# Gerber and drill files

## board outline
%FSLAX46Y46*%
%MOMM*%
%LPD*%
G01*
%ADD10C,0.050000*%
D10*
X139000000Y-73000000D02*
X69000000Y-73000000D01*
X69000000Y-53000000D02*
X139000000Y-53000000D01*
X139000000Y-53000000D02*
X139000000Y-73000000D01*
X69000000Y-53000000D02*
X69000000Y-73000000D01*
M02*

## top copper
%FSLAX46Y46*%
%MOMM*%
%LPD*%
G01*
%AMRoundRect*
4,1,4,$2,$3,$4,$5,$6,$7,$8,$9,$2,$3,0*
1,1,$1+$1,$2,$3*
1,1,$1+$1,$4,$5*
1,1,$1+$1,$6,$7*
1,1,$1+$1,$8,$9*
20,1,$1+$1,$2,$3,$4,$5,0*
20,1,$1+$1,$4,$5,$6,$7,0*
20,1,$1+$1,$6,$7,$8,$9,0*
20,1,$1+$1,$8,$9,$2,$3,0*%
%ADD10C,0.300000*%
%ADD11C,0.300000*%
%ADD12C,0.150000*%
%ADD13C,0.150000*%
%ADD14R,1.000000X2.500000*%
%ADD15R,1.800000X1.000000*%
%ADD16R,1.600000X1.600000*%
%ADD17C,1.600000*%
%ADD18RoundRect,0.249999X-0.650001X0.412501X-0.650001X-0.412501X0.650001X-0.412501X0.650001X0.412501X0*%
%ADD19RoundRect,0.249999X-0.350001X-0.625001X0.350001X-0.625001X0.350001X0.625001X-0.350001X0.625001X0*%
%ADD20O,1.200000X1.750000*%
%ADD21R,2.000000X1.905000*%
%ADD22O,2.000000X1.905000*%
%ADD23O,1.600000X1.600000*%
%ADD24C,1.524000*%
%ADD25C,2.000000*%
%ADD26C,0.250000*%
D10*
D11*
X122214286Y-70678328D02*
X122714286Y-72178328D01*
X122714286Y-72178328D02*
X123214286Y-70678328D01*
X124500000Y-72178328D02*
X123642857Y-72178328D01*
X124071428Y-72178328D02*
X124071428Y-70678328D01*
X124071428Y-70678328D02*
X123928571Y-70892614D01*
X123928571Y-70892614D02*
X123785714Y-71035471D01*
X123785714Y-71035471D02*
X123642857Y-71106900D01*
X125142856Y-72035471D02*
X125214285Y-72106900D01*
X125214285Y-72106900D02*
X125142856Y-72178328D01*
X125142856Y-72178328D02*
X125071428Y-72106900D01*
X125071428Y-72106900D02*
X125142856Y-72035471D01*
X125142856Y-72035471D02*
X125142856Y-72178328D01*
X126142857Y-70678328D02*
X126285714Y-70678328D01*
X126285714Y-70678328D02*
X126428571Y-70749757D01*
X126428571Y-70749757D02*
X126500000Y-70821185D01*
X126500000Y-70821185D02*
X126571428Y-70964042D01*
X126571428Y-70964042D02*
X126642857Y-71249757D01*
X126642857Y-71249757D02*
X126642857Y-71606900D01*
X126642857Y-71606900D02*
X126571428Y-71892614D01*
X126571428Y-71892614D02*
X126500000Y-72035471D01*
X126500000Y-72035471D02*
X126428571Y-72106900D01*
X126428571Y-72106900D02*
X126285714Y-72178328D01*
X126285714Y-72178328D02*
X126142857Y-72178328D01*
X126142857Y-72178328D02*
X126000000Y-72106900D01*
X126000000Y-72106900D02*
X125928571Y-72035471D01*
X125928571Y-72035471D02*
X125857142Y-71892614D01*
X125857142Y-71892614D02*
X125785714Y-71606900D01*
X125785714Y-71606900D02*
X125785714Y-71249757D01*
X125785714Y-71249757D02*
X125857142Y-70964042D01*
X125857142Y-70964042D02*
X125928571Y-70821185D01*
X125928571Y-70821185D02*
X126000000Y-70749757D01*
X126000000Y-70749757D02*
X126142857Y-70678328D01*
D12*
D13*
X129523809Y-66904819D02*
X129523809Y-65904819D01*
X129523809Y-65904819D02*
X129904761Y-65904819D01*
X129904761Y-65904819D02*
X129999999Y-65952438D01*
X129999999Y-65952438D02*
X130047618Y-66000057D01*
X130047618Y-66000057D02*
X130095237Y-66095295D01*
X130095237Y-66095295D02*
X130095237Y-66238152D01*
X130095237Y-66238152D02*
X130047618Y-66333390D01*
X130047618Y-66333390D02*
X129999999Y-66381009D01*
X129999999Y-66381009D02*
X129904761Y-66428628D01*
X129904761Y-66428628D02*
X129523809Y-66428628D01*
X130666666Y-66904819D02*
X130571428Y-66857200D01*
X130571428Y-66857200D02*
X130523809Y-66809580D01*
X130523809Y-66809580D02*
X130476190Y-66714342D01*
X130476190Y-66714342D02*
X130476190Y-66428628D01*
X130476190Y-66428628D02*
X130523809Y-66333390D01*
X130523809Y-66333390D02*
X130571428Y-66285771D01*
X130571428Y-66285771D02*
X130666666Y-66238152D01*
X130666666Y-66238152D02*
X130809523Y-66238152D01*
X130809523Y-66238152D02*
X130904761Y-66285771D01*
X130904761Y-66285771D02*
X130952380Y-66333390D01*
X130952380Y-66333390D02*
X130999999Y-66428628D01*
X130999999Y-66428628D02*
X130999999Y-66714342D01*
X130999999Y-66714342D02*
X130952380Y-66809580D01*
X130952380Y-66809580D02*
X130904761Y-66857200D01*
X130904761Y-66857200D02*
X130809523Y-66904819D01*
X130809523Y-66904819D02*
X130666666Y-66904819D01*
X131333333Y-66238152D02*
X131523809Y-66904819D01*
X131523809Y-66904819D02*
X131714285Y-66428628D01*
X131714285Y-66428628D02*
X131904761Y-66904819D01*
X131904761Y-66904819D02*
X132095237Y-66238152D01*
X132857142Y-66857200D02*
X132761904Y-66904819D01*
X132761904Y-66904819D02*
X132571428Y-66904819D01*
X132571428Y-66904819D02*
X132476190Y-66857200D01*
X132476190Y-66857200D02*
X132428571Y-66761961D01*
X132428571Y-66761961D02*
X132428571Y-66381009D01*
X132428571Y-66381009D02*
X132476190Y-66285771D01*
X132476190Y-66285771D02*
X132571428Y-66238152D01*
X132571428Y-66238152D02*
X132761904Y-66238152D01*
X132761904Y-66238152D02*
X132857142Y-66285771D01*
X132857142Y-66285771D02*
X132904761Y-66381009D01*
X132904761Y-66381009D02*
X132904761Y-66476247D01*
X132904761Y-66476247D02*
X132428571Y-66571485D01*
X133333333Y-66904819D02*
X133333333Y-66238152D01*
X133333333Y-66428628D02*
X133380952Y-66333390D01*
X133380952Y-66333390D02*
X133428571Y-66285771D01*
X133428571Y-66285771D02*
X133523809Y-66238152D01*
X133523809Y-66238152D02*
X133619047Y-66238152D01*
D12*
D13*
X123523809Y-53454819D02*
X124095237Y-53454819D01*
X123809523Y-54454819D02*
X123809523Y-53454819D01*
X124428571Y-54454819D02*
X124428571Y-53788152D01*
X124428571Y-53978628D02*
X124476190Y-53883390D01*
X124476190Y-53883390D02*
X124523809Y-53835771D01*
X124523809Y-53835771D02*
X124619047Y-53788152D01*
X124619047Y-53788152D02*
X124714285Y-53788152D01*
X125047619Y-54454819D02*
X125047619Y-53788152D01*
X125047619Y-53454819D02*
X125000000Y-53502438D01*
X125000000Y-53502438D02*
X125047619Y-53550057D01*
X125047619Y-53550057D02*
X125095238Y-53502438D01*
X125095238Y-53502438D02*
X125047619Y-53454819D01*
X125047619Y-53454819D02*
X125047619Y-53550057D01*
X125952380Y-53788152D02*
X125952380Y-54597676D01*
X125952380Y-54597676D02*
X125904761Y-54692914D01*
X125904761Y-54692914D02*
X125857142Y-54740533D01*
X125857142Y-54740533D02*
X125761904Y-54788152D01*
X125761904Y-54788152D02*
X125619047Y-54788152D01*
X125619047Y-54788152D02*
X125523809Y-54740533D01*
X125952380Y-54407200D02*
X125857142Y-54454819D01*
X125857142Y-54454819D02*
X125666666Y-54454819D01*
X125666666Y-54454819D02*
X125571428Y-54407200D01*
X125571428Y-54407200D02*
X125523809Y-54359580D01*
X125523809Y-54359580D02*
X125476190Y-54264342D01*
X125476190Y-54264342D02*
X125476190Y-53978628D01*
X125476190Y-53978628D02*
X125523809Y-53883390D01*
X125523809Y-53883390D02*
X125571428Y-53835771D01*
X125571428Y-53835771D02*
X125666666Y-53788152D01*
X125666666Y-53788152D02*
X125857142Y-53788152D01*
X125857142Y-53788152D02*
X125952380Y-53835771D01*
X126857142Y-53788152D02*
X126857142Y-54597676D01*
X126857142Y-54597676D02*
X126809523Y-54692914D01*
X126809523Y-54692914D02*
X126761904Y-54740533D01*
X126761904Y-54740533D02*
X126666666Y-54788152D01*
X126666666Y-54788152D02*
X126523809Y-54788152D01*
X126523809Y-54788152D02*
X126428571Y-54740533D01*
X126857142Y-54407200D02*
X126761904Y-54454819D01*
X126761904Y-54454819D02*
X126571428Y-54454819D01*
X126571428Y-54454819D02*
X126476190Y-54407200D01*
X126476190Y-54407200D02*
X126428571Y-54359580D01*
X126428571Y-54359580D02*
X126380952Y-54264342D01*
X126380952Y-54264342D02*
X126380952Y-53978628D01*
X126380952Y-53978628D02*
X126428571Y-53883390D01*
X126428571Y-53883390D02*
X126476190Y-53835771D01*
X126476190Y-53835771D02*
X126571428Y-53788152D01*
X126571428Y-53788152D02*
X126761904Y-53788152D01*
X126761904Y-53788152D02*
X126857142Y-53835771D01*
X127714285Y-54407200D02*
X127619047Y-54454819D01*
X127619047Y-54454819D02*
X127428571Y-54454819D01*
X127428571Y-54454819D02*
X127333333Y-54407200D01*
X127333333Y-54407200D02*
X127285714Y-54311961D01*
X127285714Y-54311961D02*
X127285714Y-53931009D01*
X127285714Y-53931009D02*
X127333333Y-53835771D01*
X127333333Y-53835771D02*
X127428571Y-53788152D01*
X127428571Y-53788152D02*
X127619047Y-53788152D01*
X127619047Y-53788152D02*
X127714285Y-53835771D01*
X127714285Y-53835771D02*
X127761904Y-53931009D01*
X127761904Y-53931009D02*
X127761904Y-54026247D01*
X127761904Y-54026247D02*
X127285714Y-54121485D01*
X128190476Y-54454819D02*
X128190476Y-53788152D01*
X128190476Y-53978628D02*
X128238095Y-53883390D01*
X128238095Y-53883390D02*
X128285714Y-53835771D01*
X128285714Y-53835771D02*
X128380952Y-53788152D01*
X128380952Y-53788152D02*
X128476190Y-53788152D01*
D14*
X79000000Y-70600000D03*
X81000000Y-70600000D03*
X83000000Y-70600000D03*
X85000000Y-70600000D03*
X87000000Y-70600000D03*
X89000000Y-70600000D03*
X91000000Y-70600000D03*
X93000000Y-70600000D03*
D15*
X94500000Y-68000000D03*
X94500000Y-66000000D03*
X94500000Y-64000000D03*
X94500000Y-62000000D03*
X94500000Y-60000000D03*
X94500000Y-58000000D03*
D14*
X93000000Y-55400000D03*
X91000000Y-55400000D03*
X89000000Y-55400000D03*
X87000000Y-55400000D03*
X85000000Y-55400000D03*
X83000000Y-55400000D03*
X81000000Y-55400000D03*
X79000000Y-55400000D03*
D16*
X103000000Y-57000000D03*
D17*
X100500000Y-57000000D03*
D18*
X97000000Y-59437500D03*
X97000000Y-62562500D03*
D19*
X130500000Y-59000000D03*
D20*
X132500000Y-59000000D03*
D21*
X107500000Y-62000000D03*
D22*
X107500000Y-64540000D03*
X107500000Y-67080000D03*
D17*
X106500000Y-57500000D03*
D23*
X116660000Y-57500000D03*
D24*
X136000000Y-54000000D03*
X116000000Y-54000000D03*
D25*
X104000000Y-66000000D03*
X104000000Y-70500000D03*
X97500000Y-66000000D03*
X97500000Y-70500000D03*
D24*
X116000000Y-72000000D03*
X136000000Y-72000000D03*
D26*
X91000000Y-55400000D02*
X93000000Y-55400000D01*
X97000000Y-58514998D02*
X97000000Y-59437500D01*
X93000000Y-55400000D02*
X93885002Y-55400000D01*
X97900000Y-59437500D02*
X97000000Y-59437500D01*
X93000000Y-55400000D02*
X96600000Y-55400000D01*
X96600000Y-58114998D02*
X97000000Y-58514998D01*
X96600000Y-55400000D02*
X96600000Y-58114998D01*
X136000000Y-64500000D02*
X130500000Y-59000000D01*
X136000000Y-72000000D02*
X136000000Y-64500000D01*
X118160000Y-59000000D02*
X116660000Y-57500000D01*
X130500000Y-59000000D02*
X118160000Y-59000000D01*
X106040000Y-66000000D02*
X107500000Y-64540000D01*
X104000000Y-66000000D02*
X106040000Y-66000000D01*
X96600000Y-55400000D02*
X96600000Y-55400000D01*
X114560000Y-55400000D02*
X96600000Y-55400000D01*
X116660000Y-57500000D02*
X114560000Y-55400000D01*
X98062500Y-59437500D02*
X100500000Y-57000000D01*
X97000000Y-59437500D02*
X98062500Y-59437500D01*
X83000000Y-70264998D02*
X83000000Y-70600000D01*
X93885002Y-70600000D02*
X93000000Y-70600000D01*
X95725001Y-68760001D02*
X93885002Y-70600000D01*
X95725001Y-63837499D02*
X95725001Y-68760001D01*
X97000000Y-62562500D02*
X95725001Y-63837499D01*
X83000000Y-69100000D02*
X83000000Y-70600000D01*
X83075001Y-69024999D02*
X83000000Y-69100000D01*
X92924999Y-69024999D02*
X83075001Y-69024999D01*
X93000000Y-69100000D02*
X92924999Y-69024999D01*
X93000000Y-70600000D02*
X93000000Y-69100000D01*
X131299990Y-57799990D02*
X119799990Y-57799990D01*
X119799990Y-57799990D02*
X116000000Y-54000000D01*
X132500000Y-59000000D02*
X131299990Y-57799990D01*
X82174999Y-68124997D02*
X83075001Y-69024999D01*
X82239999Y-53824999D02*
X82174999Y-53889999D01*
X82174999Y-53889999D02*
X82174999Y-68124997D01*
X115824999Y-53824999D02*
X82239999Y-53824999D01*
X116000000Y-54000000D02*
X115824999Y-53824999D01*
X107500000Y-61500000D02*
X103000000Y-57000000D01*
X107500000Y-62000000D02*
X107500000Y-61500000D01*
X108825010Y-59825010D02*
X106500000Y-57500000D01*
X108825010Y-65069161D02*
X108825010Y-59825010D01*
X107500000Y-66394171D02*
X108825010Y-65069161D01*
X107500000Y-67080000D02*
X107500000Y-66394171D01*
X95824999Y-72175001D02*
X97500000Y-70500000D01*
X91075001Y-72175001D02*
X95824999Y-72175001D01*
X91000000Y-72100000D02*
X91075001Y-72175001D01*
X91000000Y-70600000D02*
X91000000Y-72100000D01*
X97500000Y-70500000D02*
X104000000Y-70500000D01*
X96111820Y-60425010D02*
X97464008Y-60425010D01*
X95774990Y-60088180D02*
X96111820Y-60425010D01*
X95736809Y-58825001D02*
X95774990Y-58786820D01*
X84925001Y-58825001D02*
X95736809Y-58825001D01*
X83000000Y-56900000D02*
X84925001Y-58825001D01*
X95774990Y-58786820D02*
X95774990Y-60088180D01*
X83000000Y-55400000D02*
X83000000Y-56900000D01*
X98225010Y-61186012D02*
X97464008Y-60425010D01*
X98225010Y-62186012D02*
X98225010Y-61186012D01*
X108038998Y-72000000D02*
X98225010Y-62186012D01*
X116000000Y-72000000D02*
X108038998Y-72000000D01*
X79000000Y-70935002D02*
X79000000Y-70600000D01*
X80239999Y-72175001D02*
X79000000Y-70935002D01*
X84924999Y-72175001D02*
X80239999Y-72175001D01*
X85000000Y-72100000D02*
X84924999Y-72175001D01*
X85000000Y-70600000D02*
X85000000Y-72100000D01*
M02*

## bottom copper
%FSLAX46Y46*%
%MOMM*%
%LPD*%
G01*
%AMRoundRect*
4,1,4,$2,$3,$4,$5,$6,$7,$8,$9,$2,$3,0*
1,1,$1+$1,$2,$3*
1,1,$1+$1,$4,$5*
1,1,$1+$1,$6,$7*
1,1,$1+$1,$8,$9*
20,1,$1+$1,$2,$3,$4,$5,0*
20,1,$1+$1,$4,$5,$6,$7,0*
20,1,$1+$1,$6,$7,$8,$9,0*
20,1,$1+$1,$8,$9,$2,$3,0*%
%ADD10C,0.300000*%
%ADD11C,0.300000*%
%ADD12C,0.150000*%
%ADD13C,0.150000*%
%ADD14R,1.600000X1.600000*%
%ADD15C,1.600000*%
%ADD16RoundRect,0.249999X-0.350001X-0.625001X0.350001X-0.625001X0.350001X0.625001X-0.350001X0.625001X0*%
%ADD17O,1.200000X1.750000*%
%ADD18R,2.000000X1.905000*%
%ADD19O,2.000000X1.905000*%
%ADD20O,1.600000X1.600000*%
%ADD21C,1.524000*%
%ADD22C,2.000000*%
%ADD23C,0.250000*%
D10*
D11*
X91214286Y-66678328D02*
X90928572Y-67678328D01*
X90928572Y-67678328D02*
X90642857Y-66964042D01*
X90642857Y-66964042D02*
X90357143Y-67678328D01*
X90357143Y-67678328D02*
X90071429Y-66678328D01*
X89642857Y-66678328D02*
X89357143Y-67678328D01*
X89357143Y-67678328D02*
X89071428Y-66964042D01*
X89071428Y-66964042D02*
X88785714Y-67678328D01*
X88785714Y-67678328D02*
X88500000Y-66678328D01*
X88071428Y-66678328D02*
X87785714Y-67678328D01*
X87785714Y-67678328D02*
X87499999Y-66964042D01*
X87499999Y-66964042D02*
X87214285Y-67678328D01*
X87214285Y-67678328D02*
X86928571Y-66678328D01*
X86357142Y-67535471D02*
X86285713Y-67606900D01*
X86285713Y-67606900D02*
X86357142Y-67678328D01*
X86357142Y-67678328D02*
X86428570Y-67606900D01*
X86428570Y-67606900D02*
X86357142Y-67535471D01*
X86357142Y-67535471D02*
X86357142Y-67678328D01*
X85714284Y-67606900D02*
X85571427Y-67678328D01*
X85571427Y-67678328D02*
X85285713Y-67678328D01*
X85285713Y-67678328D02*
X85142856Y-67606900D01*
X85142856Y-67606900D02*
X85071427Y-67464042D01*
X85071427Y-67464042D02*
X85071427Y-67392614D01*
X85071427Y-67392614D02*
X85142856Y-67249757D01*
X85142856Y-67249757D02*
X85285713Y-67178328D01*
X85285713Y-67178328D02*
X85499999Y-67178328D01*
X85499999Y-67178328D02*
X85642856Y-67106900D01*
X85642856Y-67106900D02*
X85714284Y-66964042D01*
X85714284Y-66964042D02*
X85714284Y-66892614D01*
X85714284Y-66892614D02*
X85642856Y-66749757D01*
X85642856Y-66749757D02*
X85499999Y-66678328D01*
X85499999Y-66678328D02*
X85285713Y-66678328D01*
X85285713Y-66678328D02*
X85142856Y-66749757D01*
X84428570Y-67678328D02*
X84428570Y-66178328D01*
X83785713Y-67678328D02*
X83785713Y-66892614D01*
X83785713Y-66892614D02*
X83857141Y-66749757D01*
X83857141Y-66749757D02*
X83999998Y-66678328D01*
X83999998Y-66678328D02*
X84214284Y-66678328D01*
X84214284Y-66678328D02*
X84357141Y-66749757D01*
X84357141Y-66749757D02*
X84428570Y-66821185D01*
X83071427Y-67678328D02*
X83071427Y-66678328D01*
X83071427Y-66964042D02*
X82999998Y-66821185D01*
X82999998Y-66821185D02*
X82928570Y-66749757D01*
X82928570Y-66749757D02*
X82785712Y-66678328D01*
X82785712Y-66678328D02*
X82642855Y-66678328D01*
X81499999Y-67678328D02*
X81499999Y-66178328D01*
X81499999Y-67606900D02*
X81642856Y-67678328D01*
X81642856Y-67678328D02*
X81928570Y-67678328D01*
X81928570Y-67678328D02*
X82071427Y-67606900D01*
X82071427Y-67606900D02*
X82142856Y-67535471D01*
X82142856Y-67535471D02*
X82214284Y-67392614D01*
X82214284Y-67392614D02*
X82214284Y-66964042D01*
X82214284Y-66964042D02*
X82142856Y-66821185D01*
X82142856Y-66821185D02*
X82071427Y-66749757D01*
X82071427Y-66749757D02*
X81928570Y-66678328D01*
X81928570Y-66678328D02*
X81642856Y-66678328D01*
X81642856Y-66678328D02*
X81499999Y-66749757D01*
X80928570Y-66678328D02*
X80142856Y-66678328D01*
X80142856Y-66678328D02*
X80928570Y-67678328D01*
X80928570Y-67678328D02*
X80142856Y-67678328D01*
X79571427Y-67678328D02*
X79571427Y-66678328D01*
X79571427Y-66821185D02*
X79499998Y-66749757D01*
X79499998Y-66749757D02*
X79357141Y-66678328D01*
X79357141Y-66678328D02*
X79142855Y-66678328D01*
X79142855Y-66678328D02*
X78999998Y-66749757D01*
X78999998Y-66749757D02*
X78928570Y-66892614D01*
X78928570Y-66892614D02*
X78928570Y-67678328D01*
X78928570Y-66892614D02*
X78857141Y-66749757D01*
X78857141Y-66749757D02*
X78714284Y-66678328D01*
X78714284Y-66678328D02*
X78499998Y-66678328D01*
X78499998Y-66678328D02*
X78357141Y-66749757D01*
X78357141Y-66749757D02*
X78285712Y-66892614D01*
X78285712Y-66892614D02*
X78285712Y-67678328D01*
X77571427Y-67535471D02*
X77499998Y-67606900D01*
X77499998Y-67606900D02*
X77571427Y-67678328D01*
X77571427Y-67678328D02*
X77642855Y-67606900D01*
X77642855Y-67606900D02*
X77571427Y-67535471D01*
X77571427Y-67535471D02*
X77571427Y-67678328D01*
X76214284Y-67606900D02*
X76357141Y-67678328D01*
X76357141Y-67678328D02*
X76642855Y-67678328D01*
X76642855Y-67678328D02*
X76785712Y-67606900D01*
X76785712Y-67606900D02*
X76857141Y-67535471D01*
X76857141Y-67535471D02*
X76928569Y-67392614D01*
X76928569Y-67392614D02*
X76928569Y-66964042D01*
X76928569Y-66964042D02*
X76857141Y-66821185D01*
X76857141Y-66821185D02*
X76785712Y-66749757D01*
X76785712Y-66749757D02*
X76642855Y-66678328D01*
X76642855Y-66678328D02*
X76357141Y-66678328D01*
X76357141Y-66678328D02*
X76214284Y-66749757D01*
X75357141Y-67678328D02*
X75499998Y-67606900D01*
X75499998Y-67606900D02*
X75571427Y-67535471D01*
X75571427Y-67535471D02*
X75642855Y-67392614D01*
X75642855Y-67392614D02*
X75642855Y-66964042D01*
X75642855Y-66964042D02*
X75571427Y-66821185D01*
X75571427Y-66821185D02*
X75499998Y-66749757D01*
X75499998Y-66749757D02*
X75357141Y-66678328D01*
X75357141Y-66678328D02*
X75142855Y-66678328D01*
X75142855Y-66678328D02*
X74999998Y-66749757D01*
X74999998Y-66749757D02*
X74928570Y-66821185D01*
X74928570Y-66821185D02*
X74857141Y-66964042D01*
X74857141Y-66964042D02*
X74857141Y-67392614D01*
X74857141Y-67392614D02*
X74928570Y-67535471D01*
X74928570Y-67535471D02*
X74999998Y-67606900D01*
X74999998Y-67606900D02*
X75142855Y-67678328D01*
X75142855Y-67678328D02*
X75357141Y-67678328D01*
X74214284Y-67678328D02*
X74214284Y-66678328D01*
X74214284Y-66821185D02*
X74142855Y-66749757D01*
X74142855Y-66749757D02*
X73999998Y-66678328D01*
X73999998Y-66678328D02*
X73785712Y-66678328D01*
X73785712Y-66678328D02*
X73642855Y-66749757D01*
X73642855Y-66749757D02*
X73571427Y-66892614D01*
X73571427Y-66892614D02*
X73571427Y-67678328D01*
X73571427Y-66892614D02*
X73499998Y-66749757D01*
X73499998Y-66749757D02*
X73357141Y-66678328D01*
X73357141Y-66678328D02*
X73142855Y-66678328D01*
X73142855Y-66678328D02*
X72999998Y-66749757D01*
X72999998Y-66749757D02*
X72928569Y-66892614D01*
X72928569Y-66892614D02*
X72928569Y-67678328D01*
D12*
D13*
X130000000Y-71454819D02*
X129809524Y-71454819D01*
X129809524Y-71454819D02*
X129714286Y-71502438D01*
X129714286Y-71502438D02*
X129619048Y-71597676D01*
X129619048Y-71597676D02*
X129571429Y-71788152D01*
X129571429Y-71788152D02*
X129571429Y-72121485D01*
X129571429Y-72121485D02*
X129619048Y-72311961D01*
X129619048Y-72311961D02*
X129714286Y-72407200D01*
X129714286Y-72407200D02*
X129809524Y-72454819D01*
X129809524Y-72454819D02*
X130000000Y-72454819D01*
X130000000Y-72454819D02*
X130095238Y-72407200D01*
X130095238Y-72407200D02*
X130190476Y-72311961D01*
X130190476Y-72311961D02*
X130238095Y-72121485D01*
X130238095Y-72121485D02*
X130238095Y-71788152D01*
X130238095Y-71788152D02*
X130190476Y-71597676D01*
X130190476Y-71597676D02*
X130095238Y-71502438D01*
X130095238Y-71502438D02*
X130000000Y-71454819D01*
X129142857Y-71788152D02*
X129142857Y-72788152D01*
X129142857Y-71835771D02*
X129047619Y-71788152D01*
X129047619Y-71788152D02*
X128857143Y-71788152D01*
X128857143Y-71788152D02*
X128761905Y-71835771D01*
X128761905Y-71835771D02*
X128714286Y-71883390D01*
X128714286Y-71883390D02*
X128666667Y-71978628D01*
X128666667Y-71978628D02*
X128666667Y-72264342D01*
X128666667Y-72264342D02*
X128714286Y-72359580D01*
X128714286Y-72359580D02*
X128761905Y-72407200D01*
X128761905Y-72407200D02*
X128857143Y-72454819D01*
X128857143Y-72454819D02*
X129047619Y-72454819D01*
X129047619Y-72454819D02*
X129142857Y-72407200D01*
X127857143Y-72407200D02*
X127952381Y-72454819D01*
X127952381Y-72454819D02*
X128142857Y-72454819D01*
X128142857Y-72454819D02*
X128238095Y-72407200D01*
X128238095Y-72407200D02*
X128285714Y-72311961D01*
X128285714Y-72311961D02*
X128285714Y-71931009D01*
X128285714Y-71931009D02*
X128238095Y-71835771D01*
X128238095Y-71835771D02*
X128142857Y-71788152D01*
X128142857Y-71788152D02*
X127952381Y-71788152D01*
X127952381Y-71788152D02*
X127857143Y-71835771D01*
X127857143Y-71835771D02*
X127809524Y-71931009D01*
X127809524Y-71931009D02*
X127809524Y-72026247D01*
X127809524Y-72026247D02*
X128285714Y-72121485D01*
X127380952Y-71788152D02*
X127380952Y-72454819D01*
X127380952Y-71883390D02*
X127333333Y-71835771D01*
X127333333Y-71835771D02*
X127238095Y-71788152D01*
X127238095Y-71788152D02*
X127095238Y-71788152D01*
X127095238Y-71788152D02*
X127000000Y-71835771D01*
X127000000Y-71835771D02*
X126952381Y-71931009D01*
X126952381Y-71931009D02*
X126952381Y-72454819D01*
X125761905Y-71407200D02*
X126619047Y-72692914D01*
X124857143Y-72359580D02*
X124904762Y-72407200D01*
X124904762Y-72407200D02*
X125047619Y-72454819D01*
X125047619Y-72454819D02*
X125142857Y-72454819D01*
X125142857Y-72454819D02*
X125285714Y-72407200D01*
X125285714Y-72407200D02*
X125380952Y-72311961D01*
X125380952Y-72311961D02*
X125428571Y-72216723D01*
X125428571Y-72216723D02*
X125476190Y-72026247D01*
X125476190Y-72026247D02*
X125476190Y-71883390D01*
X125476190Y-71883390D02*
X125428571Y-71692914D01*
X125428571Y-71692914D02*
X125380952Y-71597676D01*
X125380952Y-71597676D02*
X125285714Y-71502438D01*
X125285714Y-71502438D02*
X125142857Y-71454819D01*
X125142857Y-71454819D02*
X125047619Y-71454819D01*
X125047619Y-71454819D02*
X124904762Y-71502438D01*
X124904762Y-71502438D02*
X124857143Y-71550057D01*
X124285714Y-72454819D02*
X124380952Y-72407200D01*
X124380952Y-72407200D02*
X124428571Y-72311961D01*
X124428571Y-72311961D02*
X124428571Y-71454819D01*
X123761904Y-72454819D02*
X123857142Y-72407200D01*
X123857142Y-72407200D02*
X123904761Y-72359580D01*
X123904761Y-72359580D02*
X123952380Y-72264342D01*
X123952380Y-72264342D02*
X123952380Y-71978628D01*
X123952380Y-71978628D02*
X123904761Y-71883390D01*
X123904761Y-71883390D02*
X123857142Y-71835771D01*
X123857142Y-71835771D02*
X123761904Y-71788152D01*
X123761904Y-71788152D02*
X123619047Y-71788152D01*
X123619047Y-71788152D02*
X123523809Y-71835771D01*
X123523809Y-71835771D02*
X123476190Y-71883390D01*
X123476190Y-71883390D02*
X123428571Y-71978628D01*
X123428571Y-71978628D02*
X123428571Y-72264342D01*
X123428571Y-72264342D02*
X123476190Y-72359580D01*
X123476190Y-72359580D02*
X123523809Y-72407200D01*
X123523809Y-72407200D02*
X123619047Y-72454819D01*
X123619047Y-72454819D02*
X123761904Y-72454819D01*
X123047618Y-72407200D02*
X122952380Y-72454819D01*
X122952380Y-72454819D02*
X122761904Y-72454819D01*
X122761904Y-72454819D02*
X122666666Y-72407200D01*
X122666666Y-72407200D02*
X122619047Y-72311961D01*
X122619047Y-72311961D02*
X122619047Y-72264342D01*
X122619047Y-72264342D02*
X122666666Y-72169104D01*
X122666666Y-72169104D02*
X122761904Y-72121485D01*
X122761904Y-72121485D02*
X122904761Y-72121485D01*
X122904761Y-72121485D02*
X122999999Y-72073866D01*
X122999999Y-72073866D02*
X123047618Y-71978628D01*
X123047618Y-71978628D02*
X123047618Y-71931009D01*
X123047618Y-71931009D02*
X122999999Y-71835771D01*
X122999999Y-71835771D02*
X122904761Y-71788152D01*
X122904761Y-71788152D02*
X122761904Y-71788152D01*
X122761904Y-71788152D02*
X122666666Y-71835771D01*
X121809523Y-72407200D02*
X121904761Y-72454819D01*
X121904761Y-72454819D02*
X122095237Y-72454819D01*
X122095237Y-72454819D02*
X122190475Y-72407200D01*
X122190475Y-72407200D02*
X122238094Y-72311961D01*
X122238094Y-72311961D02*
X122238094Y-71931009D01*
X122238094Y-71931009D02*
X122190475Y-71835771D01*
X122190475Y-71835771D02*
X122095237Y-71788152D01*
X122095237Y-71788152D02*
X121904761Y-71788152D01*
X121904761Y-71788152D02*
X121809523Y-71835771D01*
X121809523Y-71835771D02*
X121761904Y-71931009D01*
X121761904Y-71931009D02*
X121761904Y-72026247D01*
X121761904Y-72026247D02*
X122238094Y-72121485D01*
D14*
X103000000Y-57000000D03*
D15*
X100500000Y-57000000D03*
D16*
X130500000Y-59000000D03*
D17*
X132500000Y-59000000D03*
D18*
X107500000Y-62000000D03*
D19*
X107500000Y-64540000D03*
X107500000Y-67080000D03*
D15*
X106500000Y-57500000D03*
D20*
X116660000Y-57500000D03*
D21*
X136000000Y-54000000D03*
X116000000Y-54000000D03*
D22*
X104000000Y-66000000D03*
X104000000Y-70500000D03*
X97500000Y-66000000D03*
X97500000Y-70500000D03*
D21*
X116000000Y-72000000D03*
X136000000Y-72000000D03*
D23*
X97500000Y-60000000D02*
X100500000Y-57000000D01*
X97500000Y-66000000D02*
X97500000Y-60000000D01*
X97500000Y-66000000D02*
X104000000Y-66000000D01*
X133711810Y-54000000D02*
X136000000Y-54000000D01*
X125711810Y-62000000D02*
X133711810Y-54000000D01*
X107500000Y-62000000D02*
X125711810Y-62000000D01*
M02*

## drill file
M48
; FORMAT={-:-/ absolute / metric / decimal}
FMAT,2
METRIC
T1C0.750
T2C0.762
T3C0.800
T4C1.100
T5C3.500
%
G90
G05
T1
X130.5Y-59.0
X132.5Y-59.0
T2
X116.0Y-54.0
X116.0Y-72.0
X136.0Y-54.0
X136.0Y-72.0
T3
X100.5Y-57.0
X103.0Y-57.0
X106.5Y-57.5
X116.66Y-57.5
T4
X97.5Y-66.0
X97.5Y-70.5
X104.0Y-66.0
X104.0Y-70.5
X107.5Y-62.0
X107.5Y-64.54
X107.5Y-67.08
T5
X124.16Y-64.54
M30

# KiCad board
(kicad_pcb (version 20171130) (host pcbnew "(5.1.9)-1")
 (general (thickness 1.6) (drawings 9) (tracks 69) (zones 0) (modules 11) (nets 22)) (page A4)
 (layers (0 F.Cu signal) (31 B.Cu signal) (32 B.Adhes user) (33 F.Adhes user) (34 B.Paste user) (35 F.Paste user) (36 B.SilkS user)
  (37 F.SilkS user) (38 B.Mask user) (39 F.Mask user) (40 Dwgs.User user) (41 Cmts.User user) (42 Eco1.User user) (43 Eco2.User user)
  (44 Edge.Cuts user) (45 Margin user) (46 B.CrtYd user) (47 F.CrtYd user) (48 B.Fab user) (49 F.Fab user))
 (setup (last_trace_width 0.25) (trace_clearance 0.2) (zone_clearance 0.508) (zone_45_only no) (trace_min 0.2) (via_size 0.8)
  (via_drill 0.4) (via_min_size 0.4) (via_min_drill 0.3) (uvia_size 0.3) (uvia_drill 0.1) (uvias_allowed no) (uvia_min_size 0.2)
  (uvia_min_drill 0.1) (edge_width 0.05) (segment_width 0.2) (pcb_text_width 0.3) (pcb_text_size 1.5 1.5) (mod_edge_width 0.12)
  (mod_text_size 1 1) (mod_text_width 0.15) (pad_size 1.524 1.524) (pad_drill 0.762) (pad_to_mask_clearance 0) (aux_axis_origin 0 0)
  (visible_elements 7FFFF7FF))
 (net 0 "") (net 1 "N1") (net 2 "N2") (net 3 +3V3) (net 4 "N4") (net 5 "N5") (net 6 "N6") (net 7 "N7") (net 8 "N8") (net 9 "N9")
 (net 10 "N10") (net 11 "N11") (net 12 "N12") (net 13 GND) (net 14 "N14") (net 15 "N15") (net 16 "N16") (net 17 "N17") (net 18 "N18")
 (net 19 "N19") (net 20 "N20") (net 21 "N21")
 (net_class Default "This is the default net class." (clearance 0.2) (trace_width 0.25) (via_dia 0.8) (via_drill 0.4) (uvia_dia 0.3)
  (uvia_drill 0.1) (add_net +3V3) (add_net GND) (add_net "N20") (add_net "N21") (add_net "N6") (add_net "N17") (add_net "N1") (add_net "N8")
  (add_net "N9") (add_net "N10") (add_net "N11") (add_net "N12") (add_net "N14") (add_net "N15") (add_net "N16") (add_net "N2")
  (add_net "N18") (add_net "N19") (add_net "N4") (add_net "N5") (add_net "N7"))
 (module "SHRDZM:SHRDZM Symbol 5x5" (layer F.Cu) (at 131.5 70)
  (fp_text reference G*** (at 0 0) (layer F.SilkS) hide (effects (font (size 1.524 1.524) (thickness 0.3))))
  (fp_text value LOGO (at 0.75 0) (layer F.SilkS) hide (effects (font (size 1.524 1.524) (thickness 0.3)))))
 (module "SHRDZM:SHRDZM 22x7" (layer B.Cu) (at 83 60 180)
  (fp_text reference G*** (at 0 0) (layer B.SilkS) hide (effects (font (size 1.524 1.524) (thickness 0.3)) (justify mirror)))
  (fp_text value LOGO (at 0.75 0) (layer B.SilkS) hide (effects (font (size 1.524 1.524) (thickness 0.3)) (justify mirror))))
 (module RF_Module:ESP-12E (layer F.Cu) (at 82.5 63 90)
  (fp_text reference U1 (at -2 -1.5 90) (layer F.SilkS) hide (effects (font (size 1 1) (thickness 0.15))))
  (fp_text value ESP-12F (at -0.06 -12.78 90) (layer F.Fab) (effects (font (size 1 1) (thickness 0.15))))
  (pad 1 smd rect (at -7.6 -3.5 90) (size 2.5 1) (layers F.Cu F.Paste F.Mask) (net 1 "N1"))
  (pad 2 smd rect (at -7.6 -1.5 90) (size 2.5 1) (layers F.Cu F.Paste F.Mask) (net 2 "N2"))
  (pad 3 smd rect (at -7.6 0.5 90) (size 2.5 1) (layers F.Cu F.Paste F.Mask) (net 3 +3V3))
  (pad 4 smd rect (at -7.6 2.5 90) (size 2.5 1) (layers F.Cu F.Paste F.Mask) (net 1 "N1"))
  (pad 5 smd rect (at -7.6 4.5 90) (size 2.5 1) (layers F.Cu F.Paste F.Mask) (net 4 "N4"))
  (pad 6 smd rect (at -7.6 6.5 90) (size 2.5 1) (layers F.Cu F.Paste F.Mask) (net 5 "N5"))
  (pad 7 smd rect (at -7.6 8.5 90) (size 2.5 1) (layers F.Cu F.Paste F.Mask) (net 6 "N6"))
  (pad 8 smd rect (at -7.6 10.5 90) (size 2.5 1) (layers F.Cu F.Paste F.Mask) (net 3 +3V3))
  (pad 9 smd rect (at -5 12 90) (size 1 1.8) (layers F.Cu F.Paste F.Mask) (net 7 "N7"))
  (pad 10 smd rect (at -3 12 90) (size 1 1.8) (layers F.Cu F.Paste F.Mask) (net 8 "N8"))
  (pad 11 smd rect (at -1 12 90) (size 1 1.8) (layers F.Cu F.Paste F.Mask) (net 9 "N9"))
  (pad 12 smd rect (at 1 12 90) (size 1 1.8) (layers F.Cu F.Paste F.Mask) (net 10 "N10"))
  (pad 13 smd rect (at 3 12 90) (size 1 1.8) (layers F.Cu F.Paste F.Mask) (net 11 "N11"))
  (pad 14 smd rect (at 5 12 90) (size 1 1.8) (layers F.Cu F.Paste F.Mask) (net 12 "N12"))
  (pad 15 smd rect (at 7.6 10.5 90) (size 2.5 1) (layers F.Cu F.Paste F.Mask) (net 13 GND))
  (pad 16 smd rect (at 7.6 8.5 90) (size 2.5 1) (layers F.Cu F.Paste F.Mask) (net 13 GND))
  (pad 17 smd rect (at 7.6 6.5 90) (size 2.5 1) (layers F.Cu F.Paste F.Mask) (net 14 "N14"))
  (pad 18 smd rect (at 7.6 4.5 90) (size 2.5 1) (layers F.Cu F.Paste F.Mask) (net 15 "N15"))
  (pad 19 smd rect (at 7.6 2.5 90) (size 2.5 1) (layers F.Cu F.Paste F.Mask) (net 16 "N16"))
  (pad 20 smd rect (at 7.6 0.5 90) (size 2.5 1) (layers F.Cu F.Paste F.Mask) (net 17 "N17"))
  (pad 21 smd rect (at 7.6 -1.5 90) (size 2.5 1) (layers F.Cu F.Paste F.Mask) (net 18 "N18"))
  (pad 22 smd rect (at 7.6 -3.5 90) (size 2.5 1) (layers F.Cu F.Paste F.Mask) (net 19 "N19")))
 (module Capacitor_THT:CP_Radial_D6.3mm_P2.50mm (layer F.Cu) (at 103 57 180)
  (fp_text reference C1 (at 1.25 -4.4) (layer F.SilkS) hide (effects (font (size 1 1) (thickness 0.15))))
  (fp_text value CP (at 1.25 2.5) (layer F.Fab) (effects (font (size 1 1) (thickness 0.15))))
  (pad 1 thru_hole rect (at 0 0 180) (size 1.6 1.6) (drill 0.8) (layers *.Cu *.Mask) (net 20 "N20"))
  (pad 2 thru_hole circle (at 2.5 0 180) (size 1.6 1.6) (drill 0.8) (layers *.Cu *.Mask) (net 13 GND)))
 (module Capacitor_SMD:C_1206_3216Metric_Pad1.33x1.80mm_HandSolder (layer F.Cu) (at 97 61 270)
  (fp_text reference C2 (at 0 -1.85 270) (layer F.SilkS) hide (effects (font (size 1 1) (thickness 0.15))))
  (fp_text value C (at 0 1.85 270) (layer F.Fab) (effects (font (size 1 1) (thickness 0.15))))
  (pad 1 smd roundrect (at -1.5625 0 270) (size 1.325 1.8) (layers F.Cu F.Paste F.Mask) (roundrect_rratio 0.1886784905660377) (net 13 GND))
  (pad 2 smd roundrect (at 1.5625 0 270) (size 1.325 1.8) (layers F.Cu F.Paste F.Mask) (roundrect_rratio 0.1886784905660377) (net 3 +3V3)))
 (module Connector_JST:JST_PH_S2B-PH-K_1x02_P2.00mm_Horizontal (layer F.Cu) (at 130.5 59)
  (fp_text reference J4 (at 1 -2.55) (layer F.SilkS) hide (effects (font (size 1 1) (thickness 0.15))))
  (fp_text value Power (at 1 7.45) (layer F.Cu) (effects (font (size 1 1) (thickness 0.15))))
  (pad 1 thru_hole roundrect (at 0 0) (size 1.2 1.75) (drill 0.75) (layers *.Cu *.Mask) (roundrect_rratio 0.2083325) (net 13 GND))
  (pad 2 thru_hole oval (at 2 0) (size 1.2 1.75) (drill 0.75) (layers *.Cu *.Mask) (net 3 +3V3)))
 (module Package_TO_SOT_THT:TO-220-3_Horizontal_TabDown (layer F.Cu) (at 107.5 62 270)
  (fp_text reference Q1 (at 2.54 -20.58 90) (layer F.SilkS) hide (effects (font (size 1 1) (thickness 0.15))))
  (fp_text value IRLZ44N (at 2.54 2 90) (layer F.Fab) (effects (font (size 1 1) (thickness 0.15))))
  (pad "" np_thru_hole oval (at 2.54 -16.66 270) (size 3.5 3.5) (drill 3.5) (layers *.Cu *.Mask))
  (pad 1 thru_hole rect (at 0 0 270) (size 1.905 2) (drill 1.1) (layers *.Cu *.Mask) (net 20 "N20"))
  (pad 2 thru_hole oval (at 2.54 0 270) (size 1.905 2) (drill 1.1) (layers *.Cu *.Mask) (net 13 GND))
  (pad 3 thru_hole oval (at 5.08 0 270) (size 1.905 2) (drill 1.1) (layers *.Cu *.Mask) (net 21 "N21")))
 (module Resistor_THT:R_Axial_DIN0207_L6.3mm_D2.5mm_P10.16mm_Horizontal (layer F.Cu) (at 106.5 57.5)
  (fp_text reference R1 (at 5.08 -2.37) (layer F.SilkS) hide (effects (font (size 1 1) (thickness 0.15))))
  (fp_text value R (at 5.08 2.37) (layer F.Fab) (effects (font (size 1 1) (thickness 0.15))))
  (pad 1 thru_hole circle (at 0 0) (size 1.6 1.6) (drill 0.8) (layers *.Cu *.Mask) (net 21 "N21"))
  (pad 2 thru_hole oval (at 10.16 0) (size 1.6 1.6) (drill 0.8) (layers *.Cu *.Mask) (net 13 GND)))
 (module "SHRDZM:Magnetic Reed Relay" (layer F.Cu) (at 126 54)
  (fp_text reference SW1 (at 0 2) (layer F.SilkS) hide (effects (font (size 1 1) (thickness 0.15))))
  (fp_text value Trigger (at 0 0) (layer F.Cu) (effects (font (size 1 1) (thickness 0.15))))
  (pad 2 thru_hole circle (at 10 0) (size 1.524 1.524) (drill 0.762) (layers *.Cu *.Mask) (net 20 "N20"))
  (pad 1 thru_hole circle (at -10 0) (size 1.524 1.524) (drill 0.762) (layers *.Cu *.Mask) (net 3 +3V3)))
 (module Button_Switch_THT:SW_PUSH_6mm (layer F.Cu) (at 104 70.5 180)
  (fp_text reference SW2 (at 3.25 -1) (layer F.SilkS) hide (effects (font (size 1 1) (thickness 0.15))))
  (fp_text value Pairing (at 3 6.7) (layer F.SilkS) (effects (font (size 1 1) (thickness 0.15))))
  (pad 2 thru_hole circle (at 0 4.5 270) (size 2 2) (drill 1.1) (layers *.Cu *.Mask) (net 13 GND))
  (pad 1 thru_hole circle (at 0 0 270) (size 2 2) (drill 1.1) (layers *.Cu *.Mask) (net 6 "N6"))
  (pad 2 thru_hole circle (at 6.5 4.5 270) (size 2 2) (drill 1.1) (layers *.Cu *.Mask) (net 13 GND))
  (pad 1 thru_hole circle (at 6.5 0 270) (size 2 2) (drill 1.1) (layers *.Cu *.Mask) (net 6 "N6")))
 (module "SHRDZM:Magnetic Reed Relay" (layer B.Cu) (at 126 72)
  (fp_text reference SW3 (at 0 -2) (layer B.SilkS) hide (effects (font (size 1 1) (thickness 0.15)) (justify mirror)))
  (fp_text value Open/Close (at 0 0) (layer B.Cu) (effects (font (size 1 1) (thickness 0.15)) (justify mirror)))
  (pad 1 thru_hole circle (at -10 0) (size 1.524 1.524) (drill 0.762) (layers *.Cu *.Mask) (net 17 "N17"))
  (pad 2 thru_hole circle (at 10 0) (size 1.524 1.524) (drill 0.762) (layers *.Cu *.Mask) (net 13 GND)))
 (gr_line (start 139 73) (end 69 73) (layer Edge.Cuts) (width 0.05))
 (gr_line (start 69 53) (end 139 53) (layer Edge.Cuts) (width 0.05))
 (gr_line (start 139 53) (end 139 73) (layer Edge.Cuts) (width 0.05))
 (gr_line (start 69 53) (end 69 73) (layer Edge.Cuts) (width 0.05))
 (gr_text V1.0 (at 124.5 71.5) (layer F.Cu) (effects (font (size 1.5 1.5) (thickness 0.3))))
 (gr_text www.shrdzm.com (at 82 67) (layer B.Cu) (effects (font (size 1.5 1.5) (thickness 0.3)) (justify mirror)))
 (segment (start 91 55.4) (end 93 55.4) (width 0.25) (layer F.Cu) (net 13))
 (segment (start 97 58.514998) (end 97 59.4375) (width 0.25) (layer F.Cu) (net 13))
 (segment (start 93 55.4) (end 93.885002 55.4) (width 0.25) (layer F.Cu) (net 13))
 (segment (start 97.9 59.4375) (end 97 59.4375) (width 0.25) (layer F.Cu) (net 13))
 (segment (start 93 55.4) (end 96.6 55.4) (width 0.25) (layer F.Cu) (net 13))
 (segment (start 96.6 58.114998) (end 97 58.514998) (width 0.25) (layer F.Cu) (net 13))
 (segment (start 96.6 55.4) (end 96.6 58.114998) (width 0.25) (layer F.Cu) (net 13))
 (segment (start 136 64.5) (end 130.5 59) (width 0.25) (layer F.Cu) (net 13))
 (segment (start 136 72) (end 136 64.5) (width 0.25) (layer F.Cu) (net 13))
 (segment (start 118.16 59) (end 116.66 57.5) (width 0.25) (layer F.Cu) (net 13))
 (segment (start 130.5 59) (end 118.16 59) (width 0.25) (layer F.Cu) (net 13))
 (segment (start 106.04 66) (end 107.5 64.54) (width 0.25) (layer F.Cu) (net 13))
 (segment (start 104 66) (end 106.04 66) (width 0.25) (layer F.Cu) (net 13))
 (segment (start 96.6 55.4) (end 96.6 55.4) (width 0.25) (layer F.Cu) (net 13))
 (segment (start 114.56 55.4) (end 96.6 55.4) (width 0.25) (layer F.Cu) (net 13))
 (segment (start 116.66 57.5) (end 114.56 55.4) (width 0.25) (layer F.Cu) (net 13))
 (segment (start 97.5 60) (end 100.5 57) (width 0.25) (layer B.Cu) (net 13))
 (segment (start 97.5 66) (end 97.5 60) (width 0.25) (layer B.Cu) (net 13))
 (segment (start 97.5 66) (end 104 66) (width 0.25) (layer B.Cu) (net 13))
 (segment (start 98.0625 59.4375) (end 100.5 57) (width 0.25) (layer F.Cu) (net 13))
 (segment (start 97 59.4375) (end 98.0625 59.4375) (width 0.25) (layer F.Cu) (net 13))
 (segment (start 83 70.264998) (end 83 70.6) (width 0.25) (layer F.Cu) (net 3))
 (segment (start 93.885002 70.6) (end 93 70.6) (width 0.25) (layer F.Cu) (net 3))
 (segment (start 95.725001 68.760001) (end 93.885002 70.6) (width 0.25) (layer F.Cu) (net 3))
 (segment (start 95.725001 63.837499) (end 95.725001 68.760001) (width 0.25) (layer F.Cu) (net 3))
 (segment (start 97 62.5625) (end 95.725001 63.837499) (width 0.25) (layer F.Cu) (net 3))
 (segment (start 83 69.1) (end 83 70.6) (width 0.25) (layer F.Cu) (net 3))
 (segment (start 83.075001 69.024999) (end 83 69.1) (width 0.25) (layer F.Cu) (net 3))
 (segment (start 92.924999 69.024999) (end 83.075001 69.024999) (width 0.25) (layer F.Cu) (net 3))
 (segment (start 93 69.1) (end 92.924999 69.024999) (width 0.25) (layer F.Cu) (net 3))
 (segment (start 93 70.6) (end 93 69.1) (width 0.25) (layer F.Cu) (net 3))
 (segment (start 131.29999 57.79999) (end 119.79999 57.79999) (width 0.25) (layer F.Cu) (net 3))
 (segment (start 119.79999 57.79999) (end 116 54) (width 0.25) (layer F.Cu) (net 3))
 (segment (start 132.5 59) (end 131.29999 57.79999) (width 0.25) (layer F.Cu) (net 3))
 (segment (start 82.174999 68.124997) (end 83.075001 69.024999) (width 0.25) (layer F.Cu) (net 3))
 (segment (start 82.239999 53.824999) (end 82.174999 53.889999) (width 0.25) (layer F.Cu) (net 3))
 (segment (start 82.174999 53.889999) (end 82.174999 68.124997) (width 0.25) (layer F.Cu) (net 3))
 (segment (start 115.824999 53.824999) (end 82.239999 53.824999) (width 0.25) (layer F.Cu) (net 3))
 (segment (start 116 54) (end 115.824999 53.824999) (width 0.25) (layer F.Cu) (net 3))
 (segment (start 133.71181 54) (end 136 54) (width 0.25) (layer B.Cu) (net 20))
 (segment (start 125.71181 62) (end 133.71181 54) (width 0.25) (layer B.Cu) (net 20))
 (segment (start 107.5 62) (end 125.71181 62) (width 0.25) (layer B.Cu) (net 20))
 (segment (start 107.5 61.5) (end 103 57) (width 0.25) (layer F.Cu) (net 20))
 (segment (start 107.5 62) (end 107.5 61.5) (width 0.25) (layer F.Cu) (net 20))
 (segment (start 108.82501 59.82501) (end 106.5 57.5) (width 0.25) (layer F.Cu) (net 21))
 (segment (start 108.82501 65.069161) (end 108.82501 59.82501) (width 0.25) (layer F.Cu) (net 21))
 (segment (start 107.5 66.394171) (end 108.82501 65.069161) (width 0.25) (layer F.Cu) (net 21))
 (segment (start 107.5 67.08) (end 107.5 66.394171) (width 0.25) (layer F.Cu) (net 21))
 (segment (start 95.824999 72.175001) (end 97.5 70.5) (width 0.25) (layer F.Cu) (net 6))
 (segment (start 91.075001 72.175001) (end 95.824999 72.175001) (width 0.25) (layer F.Cu) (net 6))
 (segment (start 91 72.1) (end 91.075001 72.175001) (width 0.25) (layer F.Cu) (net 6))
 (segment (start 91 70.6) (end 91 72.1) (width 0.25) (layer F.Cu) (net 6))
 (segment (start 97.5 70.5) (end 104 70.5) (width 0.25) (layer F.Cu) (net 6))
 (segment (start 96.11182 60.42501) (end 97.464008 60.42501) (width 0.25) (layer F.Cu) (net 17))
 (segment (start 95.77499 60.08818) (end 96.11182 60.42501) (width 0.25) (layer F.Cu) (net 17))
 (segment (start 95.736809 58.825001) (end 95.77499 58.78682) (width 0.25) (layer F.Cu) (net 17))
 (segment (start 84.925001 58.825001) (end 95.736809 58.825001) (width 0.25) (layer F.Cu) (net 17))
 (segment (start 83 56.9) (end 84.925001 58.825001) (width 0.25) (layer F.Cu) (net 17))
 (segment (start 95.77499 58.78682) (end 95.77499 60.08818) (width 0.25) (layer F.Cu) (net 17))
 (segment (start 83 55.4) (end 83 56.9) (width 0.25) (layer F.Cu) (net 17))
 (segment (start 98.22501 61.186012) (end 97.464008 60.42501) (width 0.25) (layer F.Cu) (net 17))
 (segment (start 98.22501 62.186012) (end 98.22501 61.186012) (width 0.25) (layer F.Cu) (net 17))
 (segment (start 108.038998 72) (end 98.22501 62.186012) (width 0.25) (layer F.Cu) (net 17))
 (segment (start 116 72) (end 108.038998 72) (width 0.25) (layer F.Cu) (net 17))
 (segment (start 79 70.935002) (end 79 70.6) (width 0.25) (layer F.Cu) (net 1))
 (segment (start 80.239999 72.175001) (end 79 70.935002) (width 0.25) (layer F.Cu) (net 1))
 (segment (start 84.924999 72.175001) (end 80.239999 72.175001) (width 0.25) (layer F.Cu) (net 1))
 (segment (start 85 72.1) (end 84.924999 72.175001) (width 0.25) (layer F.Cu) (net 1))
 (segment (start 85 70.6) (end 85 72.1) (width 0.25) (layer F.Cu) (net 1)))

